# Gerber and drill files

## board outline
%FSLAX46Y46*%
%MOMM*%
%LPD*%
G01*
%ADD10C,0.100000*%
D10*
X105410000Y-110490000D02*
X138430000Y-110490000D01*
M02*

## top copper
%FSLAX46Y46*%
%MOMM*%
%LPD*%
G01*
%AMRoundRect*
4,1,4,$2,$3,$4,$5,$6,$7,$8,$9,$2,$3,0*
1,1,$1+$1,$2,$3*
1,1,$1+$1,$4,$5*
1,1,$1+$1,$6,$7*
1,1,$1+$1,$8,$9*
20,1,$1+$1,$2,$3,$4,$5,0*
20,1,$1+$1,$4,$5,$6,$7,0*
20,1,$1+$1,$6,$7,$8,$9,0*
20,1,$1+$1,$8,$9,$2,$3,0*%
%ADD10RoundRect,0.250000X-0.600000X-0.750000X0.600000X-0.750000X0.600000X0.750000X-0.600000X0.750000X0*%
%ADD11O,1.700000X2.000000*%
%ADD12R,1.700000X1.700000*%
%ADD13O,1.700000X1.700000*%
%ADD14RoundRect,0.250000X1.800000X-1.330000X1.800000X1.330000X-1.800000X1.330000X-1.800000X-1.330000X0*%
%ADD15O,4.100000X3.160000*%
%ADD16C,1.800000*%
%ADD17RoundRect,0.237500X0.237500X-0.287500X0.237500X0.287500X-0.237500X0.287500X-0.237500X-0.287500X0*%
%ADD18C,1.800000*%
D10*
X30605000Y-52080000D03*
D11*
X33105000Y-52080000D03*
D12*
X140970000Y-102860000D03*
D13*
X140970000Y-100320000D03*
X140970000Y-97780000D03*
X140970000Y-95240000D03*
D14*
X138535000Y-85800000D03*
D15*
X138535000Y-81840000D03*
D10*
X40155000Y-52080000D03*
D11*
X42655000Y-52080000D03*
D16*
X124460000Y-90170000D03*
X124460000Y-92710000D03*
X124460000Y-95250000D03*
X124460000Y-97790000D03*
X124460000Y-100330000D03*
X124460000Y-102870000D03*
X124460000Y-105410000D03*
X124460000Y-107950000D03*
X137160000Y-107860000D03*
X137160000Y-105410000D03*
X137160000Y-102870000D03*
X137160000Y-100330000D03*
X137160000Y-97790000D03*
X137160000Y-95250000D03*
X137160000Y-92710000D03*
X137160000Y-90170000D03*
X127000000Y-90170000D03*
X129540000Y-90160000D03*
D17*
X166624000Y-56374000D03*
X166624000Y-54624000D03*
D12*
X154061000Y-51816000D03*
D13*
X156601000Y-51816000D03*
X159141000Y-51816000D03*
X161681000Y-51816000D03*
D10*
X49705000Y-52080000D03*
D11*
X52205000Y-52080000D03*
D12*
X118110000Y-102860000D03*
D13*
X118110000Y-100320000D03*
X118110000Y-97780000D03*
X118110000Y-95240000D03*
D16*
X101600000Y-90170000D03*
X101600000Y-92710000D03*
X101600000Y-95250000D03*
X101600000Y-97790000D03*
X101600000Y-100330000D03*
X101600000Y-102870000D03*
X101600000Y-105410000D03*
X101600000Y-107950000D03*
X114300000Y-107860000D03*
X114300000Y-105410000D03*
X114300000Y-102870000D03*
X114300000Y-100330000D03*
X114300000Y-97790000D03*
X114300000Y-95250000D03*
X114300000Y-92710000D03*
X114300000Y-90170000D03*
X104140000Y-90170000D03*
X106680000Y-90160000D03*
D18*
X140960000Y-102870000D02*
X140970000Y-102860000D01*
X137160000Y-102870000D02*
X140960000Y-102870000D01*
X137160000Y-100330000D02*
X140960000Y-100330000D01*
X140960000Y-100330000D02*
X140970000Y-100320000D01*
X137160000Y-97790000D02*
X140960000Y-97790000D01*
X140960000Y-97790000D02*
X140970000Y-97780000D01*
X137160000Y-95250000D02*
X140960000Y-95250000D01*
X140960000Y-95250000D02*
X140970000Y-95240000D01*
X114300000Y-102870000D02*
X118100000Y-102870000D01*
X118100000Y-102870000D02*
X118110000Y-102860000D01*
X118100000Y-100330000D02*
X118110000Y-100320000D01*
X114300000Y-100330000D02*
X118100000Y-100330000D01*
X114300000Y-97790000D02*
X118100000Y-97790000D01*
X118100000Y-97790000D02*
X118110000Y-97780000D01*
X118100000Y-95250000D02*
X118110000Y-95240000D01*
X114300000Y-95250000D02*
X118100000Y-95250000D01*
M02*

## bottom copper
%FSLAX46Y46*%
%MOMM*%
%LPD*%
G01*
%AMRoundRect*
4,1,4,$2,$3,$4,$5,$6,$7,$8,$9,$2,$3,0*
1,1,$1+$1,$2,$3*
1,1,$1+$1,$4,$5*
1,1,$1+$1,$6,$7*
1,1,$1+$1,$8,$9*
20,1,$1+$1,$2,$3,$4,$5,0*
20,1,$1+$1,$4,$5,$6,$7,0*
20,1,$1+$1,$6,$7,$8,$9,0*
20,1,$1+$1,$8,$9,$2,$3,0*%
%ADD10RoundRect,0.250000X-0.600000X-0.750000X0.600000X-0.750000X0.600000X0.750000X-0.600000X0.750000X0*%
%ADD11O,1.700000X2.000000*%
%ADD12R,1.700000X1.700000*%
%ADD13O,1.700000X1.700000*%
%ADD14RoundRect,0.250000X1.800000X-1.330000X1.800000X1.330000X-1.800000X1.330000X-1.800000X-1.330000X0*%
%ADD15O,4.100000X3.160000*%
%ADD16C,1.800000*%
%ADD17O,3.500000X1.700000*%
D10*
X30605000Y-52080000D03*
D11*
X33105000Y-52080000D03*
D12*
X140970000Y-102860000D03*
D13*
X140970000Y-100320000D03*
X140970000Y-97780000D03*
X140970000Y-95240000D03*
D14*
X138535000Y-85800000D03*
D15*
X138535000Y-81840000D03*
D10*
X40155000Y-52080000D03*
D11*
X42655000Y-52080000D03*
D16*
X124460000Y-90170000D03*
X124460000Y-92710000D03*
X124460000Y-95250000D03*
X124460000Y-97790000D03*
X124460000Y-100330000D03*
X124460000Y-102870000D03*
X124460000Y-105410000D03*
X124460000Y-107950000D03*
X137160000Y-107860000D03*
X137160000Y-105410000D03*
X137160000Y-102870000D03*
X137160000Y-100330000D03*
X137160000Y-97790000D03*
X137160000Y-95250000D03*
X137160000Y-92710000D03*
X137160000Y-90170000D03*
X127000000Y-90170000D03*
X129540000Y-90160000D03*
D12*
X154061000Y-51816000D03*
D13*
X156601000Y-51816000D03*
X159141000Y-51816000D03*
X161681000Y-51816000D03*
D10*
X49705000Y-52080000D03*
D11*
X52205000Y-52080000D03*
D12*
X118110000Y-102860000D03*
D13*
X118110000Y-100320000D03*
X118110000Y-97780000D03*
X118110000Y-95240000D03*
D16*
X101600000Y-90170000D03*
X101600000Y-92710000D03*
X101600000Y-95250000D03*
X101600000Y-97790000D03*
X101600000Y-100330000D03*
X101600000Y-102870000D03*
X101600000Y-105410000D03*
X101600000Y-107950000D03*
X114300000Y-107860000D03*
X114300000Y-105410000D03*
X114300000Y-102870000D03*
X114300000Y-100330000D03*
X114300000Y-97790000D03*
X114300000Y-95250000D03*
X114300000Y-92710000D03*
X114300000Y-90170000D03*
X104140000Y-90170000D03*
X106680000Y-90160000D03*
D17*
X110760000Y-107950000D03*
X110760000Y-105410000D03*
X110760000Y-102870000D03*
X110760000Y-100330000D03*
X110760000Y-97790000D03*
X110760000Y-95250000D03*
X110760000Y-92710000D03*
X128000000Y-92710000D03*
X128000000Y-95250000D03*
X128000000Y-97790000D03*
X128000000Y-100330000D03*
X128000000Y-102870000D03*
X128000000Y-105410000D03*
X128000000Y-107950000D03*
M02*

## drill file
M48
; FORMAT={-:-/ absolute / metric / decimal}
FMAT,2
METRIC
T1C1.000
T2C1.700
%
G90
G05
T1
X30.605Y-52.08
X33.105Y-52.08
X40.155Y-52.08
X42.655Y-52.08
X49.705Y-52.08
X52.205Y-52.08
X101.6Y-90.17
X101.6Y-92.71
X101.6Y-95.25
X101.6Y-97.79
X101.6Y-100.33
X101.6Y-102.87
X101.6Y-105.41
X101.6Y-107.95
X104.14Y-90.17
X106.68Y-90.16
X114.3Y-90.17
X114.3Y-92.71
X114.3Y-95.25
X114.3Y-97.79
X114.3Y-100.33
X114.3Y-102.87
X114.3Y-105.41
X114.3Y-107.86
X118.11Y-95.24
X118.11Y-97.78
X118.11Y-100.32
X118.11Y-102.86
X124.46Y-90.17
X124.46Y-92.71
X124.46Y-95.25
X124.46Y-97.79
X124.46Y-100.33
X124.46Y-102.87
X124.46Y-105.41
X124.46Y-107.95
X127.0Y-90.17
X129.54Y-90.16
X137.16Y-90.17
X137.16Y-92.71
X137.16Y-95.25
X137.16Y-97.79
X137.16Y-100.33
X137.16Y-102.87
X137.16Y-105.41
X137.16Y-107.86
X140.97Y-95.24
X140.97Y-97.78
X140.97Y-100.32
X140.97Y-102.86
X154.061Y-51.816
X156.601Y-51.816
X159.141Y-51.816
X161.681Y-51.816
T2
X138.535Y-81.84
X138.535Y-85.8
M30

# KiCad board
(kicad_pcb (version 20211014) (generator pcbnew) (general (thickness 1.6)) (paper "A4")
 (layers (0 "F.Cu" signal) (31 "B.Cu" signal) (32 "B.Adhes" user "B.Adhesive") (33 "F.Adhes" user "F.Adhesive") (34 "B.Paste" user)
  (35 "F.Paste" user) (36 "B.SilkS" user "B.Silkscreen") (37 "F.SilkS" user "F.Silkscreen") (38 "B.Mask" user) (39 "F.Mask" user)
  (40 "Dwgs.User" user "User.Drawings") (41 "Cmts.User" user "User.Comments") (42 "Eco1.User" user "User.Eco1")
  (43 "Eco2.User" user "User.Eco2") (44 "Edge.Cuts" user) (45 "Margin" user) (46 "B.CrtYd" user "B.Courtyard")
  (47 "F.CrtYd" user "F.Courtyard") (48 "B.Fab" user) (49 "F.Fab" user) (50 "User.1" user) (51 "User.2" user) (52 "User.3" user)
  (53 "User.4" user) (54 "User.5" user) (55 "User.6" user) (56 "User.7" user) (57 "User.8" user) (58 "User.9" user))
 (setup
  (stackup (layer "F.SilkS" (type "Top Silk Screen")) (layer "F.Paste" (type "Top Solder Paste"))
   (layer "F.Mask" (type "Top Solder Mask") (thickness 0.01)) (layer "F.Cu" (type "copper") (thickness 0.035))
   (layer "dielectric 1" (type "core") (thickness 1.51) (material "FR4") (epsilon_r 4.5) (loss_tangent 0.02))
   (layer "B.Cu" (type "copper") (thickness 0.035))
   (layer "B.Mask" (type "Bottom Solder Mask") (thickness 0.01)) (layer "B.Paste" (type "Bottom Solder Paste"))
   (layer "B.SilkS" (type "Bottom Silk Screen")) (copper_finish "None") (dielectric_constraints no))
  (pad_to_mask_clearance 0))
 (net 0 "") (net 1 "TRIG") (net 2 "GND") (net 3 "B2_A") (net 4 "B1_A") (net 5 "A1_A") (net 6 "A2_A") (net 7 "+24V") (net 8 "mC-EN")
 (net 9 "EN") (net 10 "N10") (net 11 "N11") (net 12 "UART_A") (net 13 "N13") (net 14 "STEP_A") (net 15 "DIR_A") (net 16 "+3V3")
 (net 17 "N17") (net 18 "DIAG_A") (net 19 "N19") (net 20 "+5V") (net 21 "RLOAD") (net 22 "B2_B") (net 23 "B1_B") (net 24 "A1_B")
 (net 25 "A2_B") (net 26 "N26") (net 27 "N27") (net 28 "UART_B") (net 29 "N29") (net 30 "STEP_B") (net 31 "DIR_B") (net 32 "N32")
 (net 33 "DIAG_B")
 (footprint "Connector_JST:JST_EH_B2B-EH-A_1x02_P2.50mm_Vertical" (layer "F.Cu") (at 30.605 52.08)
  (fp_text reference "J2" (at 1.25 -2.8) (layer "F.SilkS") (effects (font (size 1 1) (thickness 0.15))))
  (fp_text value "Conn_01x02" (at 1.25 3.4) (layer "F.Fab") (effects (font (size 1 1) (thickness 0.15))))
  (pad "1" thru_hole roundrect locked (at 0 0) (size 1.7 2) (drill 1) (layers *.Cu *.Mask) (roundrect_rratio 0.147059) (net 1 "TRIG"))
  (pad "2" thru_hole oval locked (at 2.5 0) (size 1.7 2) (drill 1) (layers *.Cu *.Mask) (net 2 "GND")))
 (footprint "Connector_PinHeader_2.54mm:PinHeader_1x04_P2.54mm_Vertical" (layer "F.Cu") (at 140.97 102.86 180)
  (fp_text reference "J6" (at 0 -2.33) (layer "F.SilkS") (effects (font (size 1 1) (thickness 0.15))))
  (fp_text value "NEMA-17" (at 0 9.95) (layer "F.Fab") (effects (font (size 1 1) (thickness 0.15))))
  (pad "1" thru_hole rect locked (at 0 0 180) (size 1.7 1.7) (drill 1) (layers *.Cu *.Mask) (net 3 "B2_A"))
  (pad "2" thru_hole oval locked (at 0 2.54 180) (size 1.7 1.7) (drill 1) (layers *.Cu *.Mask) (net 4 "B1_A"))
  (pad "3" thru_hole oval locked (at 0 5.08 180) (size 1.7 1.7) (drill 1) (layers *.Cu *.Mask) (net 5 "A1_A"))
  (pad "4" thru_hole oval locked (at 0 7.62 180) (size 1.7 1.7) (drill 1) (layers *.Cu *.Mask) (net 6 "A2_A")))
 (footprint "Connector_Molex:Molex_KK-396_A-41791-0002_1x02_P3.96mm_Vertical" (layer "F.Cu") (at 138.535 85.8 90)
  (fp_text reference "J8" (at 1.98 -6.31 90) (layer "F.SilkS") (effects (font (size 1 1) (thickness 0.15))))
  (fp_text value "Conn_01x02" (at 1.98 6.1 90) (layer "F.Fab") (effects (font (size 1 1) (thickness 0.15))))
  (pad "1" thru_hole roundrect locked (at 0 0 90) (size 3.16 4.1) (drill 1.7) (layers *.Cu *.Mask) (roundrect_rratio 0.079114)
   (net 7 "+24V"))
  (pad "2" thru_hole oval locked (at 3.96 0 90) (size 3.16 4.1) (drill 1.7) (layers *.Cu *.Mask) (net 2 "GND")))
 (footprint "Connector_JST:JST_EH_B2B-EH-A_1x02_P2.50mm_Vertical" (layer "F.Cu") (at 40.155 52.08)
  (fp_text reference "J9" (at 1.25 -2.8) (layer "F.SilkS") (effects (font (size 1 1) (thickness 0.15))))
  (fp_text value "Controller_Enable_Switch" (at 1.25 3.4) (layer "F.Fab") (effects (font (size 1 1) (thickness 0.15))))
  (pad "1" thru_hole roundrect locked (at 0 0) (size 1.7 2) (drill 1) (layers *.Cu *.Mask) (roundrect_rratio 0.147059) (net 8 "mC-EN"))
  (pad "2" thru_hole oval locked (at 2.5 0) (size 1.7 2) (drill 1) (layers *.Cu *.Mask) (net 2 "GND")))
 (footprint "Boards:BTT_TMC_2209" (layer "F.Cu") (at 130.81 99.06)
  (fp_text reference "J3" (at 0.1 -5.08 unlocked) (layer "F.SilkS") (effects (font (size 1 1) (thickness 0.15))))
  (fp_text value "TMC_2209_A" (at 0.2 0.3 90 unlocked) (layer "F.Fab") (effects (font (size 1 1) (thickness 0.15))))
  (pad "1" thru_hole circle (at -6.35 -8.89) (size 1.8 1.8) (drill 1) (layers *.Cu *.Mask) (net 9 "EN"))
  (pad "2" thru_hole circle (at -6.35 -6.35) (size 1.8 1.8) (drill 1) (layers *.Cu *.Mask) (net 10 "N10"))
  (pad "3" thru_hole circle (at -6.35 -3.81) (size 1.8 1.8) (drill 1) (layers *.Cu *.Mask) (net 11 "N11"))
  (pad "4" thru_hole circle (at -6.35 -1.27) (size 1.8 1.8) (drill 1) (layers *.Cu *.Mask) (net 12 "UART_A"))
  (pad "5" thru_hole circle (at -6.35 1.27) (size 1.8 1.8) (drill 1) (layers *.Cu *.Mask) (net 12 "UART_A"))
  (pad "6" thru_hole circle (at -6.35 3.81) (size 1.8 1.8) (drill 1) (layers *.Cu *.Mask) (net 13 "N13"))
  (pad "7" thru_hole circle (at -6.35 6.35) (size 1.8 1.8) (drill 1) (layers *.Cu *.Mask) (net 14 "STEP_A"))
  (pad "8" thru_hole circle (at -6.35 8.89) (size 1.8 1.8) (drill 1) (layers *.Cu *.Mask) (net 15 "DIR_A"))
  (pad "9" thru_hole circle (at 6.35 8.8) (size 1.8 1.8) (drill 1) (layers *.Cu *.Mask) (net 2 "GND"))
  (pad "10" thru_hole circle (at 6.35 6.35) (size 1.8 1.8) (drill 1) (layers *.Cu *.Mask) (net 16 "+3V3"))
  (pad "11" thru_hole circle (at 6.35 3.81) (size 1.8 1.8) (drill 1) (layers *.Cu *.Mask) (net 3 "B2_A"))
  (pad "12" thru_hole circle (at 6.35 1.27) (size 1.8 1.8) (drill 1) (layers *.Cu *.Mask) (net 4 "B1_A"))
  (pad "13" thru_hole circle (at 6.35 -1.27) (size 1.8 1.8) (drill 1) (layers *.Cu *.Mask) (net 5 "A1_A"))
  (pad "14" thru_hole circle (at 6.35 -3.81) (size 1.8 1.8) (drill 1) (layers *.Cu *.Mask) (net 6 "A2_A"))
  (pad "15" thru_hole circle (at 6.35 -6.35) (size 1.8 1.8) (drill 1) (layers *.Cu *.Mask) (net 2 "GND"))
  (pad "16" thru_hole circle (at 6.35 -8.89) (size 1.8 1.8) (drill 1) (layers *.Cu *.Mask) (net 7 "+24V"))
  (pad "17" thru_hole circle (at -3.81 -8.89) (size 1.8 1.8) (drill 1) (layers *.Cu *.Mask) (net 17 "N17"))
  (pad "18" thru_hole circle (at -1.27 -8.9) (size 1.8 1.8) (drill 1) (layers *.Cu *.Mask) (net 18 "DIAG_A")))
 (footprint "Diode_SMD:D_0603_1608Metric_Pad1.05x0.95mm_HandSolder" (layer "F.Cu") (at 166.624 55.499 90)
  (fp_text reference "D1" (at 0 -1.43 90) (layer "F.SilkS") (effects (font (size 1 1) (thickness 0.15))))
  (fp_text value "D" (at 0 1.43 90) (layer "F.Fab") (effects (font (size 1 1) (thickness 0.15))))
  (pad "1" smd roundrect locked (at -0.875 0 90) (size 1.05 0.95) (layers "F.Cu" "F.Paste" "F.Mask") (roundrect_rratio 0.25) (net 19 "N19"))
  (pad "2" smd roundrect locked (at 0.875 0 90) (size 1.05 0.95) (layers "F.Cu" "F.Paste" "F.Mask") (roundrect_rratio 0.25) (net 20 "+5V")))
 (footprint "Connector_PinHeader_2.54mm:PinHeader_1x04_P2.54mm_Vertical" (layer "F.Cu") (at 154.061 51.816 90)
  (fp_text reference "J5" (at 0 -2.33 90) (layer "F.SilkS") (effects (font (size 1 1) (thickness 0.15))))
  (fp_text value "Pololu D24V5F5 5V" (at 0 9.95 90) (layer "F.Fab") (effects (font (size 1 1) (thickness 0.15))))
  (pad "1" thru_hole rect locked (at 0 0 90) (size 1.7 1.7) (drill 1) (layers *.Cu *.Mask) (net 8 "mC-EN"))
  (pad "2" thru_hole oval locked (at 0 2.54 90) (size 1.7 1.7) (drill 1) (layers *.Cu *.Mask) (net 7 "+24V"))
  (pad "3" thru_hole oval locked (at 0 5.08 90) (size 1.7 1.7) (drill 1) (layers *.Cu *.Mask) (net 2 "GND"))
  (pad "4" thru_hole oval locked (at 0 7.62 90) (size 1.7 1.7) (drill 1) (layers *.Cu *.Mask) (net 20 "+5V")))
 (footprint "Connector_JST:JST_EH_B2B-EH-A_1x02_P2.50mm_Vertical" (layer "F.Cu") (at 49.705 52.08)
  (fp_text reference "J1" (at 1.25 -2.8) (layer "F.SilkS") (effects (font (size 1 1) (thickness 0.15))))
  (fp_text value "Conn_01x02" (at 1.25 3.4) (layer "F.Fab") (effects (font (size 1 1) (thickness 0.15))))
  (pad "1" thru_hole roundrect locked (at 0 0) (size 1.7 2) (drill 1) (layers *.Cu *.Mask) (roundrect_rratio 0.147059) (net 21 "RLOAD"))
  (pad "2" thru_hole oval locked (at 2.5 0) (size 1.7 2) (drill 1) (layers *.Cu *.Mask) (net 2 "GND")))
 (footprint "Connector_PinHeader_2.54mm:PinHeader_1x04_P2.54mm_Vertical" (layer "F.Cu") (at 118.11 102.86 180)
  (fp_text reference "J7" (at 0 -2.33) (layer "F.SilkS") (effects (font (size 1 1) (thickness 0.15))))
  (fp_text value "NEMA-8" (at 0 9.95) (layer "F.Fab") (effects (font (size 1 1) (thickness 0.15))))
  (pad "1" thru_hole rect locked (at 0 0 180) (size 1.7 1.7) (drill 1) (layers *.Cu *.Mask) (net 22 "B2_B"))
  (pad "2" thru_hole oval locked (at 0 2.54 180) (size 1.7 1.7) (drill 1) (layers *.Cu *.Mask) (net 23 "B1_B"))
  (pad "3" thru_hole oval locked (at 0 5.08 180) (size 1.7 1.7) (drill 1) (layers *.Cu *.Mask) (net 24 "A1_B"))
  (pad "4" thru_hole oval locked (at 0 7.62 180) (size 1.7 1.7) (drill 1) (layers *.Cu *.Mask) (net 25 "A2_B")))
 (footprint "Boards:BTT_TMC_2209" (layer "F.Cu") (at 107.95 99.06)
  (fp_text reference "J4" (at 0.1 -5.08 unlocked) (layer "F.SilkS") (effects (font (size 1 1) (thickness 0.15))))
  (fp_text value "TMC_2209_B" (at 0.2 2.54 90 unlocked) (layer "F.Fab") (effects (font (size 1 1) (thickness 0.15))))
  (pad "1" thru_hole circle (at -6.35 -8.89) (size 1.8 1.8) (drill 1) (layers *.Cu *.Mask) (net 9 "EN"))
  (pad "2" thru_hole circle (at -6.35 -6.35) (size 1.8 1.8) (drill 1) (layers *.Cu *.Mask) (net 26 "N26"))
  (pad "3" thru_hole circle (at -6.35 -3.81) (size 1.8 1.8) (drill 1) (layers *.Cu *.Mask) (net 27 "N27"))
  (pad "4" thru_hole circle (at -6.35 -1.27) (size 1.8 1.8) (drill 1) (layers *.Cu *.Mask) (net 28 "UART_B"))
  (pad "5" thru_hole circle (at -6.35 1.27) (size 1.8 1.8) (drill 1) (layers *.Cu *.Mask) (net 28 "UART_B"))
  (pad "6" thru_hole circle (at -6.35 3.81) (size 1.8 1.8) (drill 1) (layers *.Cu *.Mask) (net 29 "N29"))
  (pad "7" thru_hole circle (at -6.35 6.35) (size 1.8 1.8) (drill 1) (layers *.Cu *.Mask) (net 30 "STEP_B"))
  (pad "8" thru_hole circle (at -6.35 8.89) (size 1.8 1.8) (drill 1) (layers *.Cu *.Mask) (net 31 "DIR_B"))
  (pad "9" thru_hole circle (at 6.35 8.8) (size 1.8 1.8) (drill 1) (layers *.Cu *.Mask) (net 2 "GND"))
  (pad "10" thru_hole circle (at 6.35 6.35) (size 1.8 1.8) (drill 1) (layers *.Cu *.Mask) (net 16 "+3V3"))
  (pad "11" thru_hole circle (at 6.35 3.81) (size 1.8 1.8) (drill 1) (layers *.Cu *.Mask) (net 22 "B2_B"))
  (pad "12" thru_hole circle (at 6.35 1.27) (size 1.8 1.8) (drill 1) (layers *.Cu *.Mask) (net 23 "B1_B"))
  (pad "13" thru_hole circle (at 6.35 -1.27) (size 1.8 1.8) (drill 1) (layers *.Cu *.Mask) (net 24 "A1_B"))
  (pad "14" thru_hole circle (at 6.35 -3.81) (size 1.8 1.8) (drill 1) (layers *.Cu *.Mask) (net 25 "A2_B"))
  (pad "15" thru_hole circle (at 6.35 -6.35) (size 1.8 1.8) (drill 1) (layers *.Cu *.Mask) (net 2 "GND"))
  (pad "16" thru_hole circle (at 6.35 -8.89) (size 1.8 1.8) (drill 1) (layers *.Cu *.Mask) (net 7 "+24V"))
  (pad "17" thru_hole circle (at -3.81 -8.89) (size 1.8 1.8) (drill 1) (layers *.Cu *.Mask) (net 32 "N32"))
  (pad "18" thru_hole circle (at -1.27 -8.9) (size 1.8 1.8) (drill 1) (layers *.Cu *.Mask) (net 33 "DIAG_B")))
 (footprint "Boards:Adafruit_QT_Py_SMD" (layer "B.Cu") (at 119.38 100.33)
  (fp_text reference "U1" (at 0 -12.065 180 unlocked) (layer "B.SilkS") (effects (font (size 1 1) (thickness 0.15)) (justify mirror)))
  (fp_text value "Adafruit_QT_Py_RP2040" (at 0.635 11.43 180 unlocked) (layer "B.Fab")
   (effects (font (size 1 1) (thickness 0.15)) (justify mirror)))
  (pad "1" smd oval (at -7.62 7.62 180) (size 3.5 1.7) (drill (offset 1 0)) (layers "B.Cu" "B.Paste" "B.Mask") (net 9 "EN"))
  (pad "2" smd oval (at -7.62 5.08 180) (size 3.5 1.7) (drill (offset 1 0)) (layers "B.Cu" "B.Paste" "B.Mask") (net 28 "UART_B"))
  (pad "3" smd oval (at -7.62 2.54 180) (size 3.5 1.7) (drill (offset 1 0)) (layers "B.Cu" "B.Paste" "B.Mask") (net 33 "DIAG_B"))
  (pad "4" smd oval (at -7.62 0 180) (size 3.5 1.7) (drill (offset 1 0)) (layers "B.Cu" "B.Paste" "B.Mask") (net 31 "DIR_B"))
  (pad "5" smd oval (at -7.62 -2.54 180) (size 3.5 1.7) (drill (offset 1 0)) (layers "B.Cu" "B.Paste" "B.Mask") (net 15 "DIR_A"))
  (pad "6" smd oval (at -7.62 -5.08 180) (size 3.5 1.7) (drill (offset 1 0)) (layers "B.Cu" "B.Paste" "B.Mask") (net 14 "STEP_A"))
  (pad "7" smd oval (at -7.62 -7.62 180) (size 3.5 1.7) (drill (offset 1 0)) (layers "B.Cu" "B.Paste" "B.Mask") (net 12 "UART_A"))
  (pad "8" smd oval (at 7.62 -7.62) (size 3.5 1.7) (drill (offset 1 0)) (layers "B.Cu" "B.Paste" "B.Mask") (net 18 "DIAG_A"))
  (pad "9" smd oval (at 7.62 -5.08) (size 3.5 1.7) (drill (offset 1 0)) (layers "B.Cu" "B.Paste" "B.Mask") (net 30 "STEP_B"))
  (pad "10" smd oval (at 7.62 -2.54) (size 3.5 1.7) (drill (offset 1 0)) (layers "B.Cu" "B.Paste" "B.Mask") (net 1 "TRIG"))
  (pad "11" smd oval (at 7.62 0) (size 3.5 1.7) (drill (offset 1 0)) (layers "B.Cu" "B.Paste" "B.Mask") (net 21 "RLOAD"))
  (pad "12" smd oval (at 7.62 2.54) (size 3.5 1.7) (drill (offset 1 0)) (layers "B.Cu" "B.Paste" "B.Mask") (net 16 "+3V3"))
  (pad "13" smd oval (at 7.62 5.08) (size 3.5 1.7) (drill (offset 1 0)) (layers "B.Cu" "B.Paste" "B.Mask") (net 2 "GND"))
  (pad "14" smd oval (at 7.62 7.62) (size 3.5 1.7) (drill (offset 1 0)) (layers "B.Cu" "B.Paste" "B.Mask") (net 19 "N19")))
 (gr_line (start 105.41 110.49) (end 138.43 110.49) (layer "Edge.Cuts") (width 0.1))
 (segment (start 140.96 102.87) (end 140.97 102.86) (width 1.8) (layer "F.Cu") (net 3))
 (segment (start 137.16 102.87) (end 140.96 102.87) (width 1.8) (layer "F.Cu") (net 3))
 (segment (start 137.16 100.33) (end 140.96 100.33) (width 1.8) (layer "F.Cu") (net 4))
 (segment (start 140.96 100.33) (end 140.97 100.32) (width 1.8) (layer "F.Cu") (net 4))
 (segment (start 137.16 97.79) (end 140.96 97.79) (width 1.8) (layer "F.Cu") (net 5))
 (segment (start 140.96 97.79) (end 140.97 97.78) (width 1.8) (layer "F.Cu") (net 5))
 (segment (start 137.16 95.25) (end 140.96 95.25) (width 1.8) (layer "F.Cu") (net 6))
 (segment (start 140.96 95.25) (end 140.97 95.24) (width 1.8) (layer "F.Cu") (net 6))
 (segment (start 114.3 102.87) (end 118.1 102.87) (width 1.8) (layer "F.Cu") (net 22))
 (segment (start 118.1 102.87) (end 118.11 102.86) (width 1.8) (layer "F.Cu") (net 22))
 (segment (start 118.1 100.33) (end 118.11 100.32) (width 1.8) (layer "F.Cu") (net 23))
 (segment (start 114.3 100.33) (end 118.1 100.33) (width 1.8) (layer "F.Cu") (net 23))
 (segment (start 114.3 97.79) (end 118.1 97.79) (width 1.8) (layer "F.Cu") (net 24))
 (segment (start 118.1 97.79) (end 118.11 97.78) (width 1.8) (layer "F.Cu") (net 24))
 (segment (start 118.1 95.25) (end 118.11 95.24) (width 1.8) (layer "F.Cu") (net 25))
 (segment (start 114.3 95.25) (end 118.1 95.25) (width 1.8) (layer "F.Cu") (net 25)))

